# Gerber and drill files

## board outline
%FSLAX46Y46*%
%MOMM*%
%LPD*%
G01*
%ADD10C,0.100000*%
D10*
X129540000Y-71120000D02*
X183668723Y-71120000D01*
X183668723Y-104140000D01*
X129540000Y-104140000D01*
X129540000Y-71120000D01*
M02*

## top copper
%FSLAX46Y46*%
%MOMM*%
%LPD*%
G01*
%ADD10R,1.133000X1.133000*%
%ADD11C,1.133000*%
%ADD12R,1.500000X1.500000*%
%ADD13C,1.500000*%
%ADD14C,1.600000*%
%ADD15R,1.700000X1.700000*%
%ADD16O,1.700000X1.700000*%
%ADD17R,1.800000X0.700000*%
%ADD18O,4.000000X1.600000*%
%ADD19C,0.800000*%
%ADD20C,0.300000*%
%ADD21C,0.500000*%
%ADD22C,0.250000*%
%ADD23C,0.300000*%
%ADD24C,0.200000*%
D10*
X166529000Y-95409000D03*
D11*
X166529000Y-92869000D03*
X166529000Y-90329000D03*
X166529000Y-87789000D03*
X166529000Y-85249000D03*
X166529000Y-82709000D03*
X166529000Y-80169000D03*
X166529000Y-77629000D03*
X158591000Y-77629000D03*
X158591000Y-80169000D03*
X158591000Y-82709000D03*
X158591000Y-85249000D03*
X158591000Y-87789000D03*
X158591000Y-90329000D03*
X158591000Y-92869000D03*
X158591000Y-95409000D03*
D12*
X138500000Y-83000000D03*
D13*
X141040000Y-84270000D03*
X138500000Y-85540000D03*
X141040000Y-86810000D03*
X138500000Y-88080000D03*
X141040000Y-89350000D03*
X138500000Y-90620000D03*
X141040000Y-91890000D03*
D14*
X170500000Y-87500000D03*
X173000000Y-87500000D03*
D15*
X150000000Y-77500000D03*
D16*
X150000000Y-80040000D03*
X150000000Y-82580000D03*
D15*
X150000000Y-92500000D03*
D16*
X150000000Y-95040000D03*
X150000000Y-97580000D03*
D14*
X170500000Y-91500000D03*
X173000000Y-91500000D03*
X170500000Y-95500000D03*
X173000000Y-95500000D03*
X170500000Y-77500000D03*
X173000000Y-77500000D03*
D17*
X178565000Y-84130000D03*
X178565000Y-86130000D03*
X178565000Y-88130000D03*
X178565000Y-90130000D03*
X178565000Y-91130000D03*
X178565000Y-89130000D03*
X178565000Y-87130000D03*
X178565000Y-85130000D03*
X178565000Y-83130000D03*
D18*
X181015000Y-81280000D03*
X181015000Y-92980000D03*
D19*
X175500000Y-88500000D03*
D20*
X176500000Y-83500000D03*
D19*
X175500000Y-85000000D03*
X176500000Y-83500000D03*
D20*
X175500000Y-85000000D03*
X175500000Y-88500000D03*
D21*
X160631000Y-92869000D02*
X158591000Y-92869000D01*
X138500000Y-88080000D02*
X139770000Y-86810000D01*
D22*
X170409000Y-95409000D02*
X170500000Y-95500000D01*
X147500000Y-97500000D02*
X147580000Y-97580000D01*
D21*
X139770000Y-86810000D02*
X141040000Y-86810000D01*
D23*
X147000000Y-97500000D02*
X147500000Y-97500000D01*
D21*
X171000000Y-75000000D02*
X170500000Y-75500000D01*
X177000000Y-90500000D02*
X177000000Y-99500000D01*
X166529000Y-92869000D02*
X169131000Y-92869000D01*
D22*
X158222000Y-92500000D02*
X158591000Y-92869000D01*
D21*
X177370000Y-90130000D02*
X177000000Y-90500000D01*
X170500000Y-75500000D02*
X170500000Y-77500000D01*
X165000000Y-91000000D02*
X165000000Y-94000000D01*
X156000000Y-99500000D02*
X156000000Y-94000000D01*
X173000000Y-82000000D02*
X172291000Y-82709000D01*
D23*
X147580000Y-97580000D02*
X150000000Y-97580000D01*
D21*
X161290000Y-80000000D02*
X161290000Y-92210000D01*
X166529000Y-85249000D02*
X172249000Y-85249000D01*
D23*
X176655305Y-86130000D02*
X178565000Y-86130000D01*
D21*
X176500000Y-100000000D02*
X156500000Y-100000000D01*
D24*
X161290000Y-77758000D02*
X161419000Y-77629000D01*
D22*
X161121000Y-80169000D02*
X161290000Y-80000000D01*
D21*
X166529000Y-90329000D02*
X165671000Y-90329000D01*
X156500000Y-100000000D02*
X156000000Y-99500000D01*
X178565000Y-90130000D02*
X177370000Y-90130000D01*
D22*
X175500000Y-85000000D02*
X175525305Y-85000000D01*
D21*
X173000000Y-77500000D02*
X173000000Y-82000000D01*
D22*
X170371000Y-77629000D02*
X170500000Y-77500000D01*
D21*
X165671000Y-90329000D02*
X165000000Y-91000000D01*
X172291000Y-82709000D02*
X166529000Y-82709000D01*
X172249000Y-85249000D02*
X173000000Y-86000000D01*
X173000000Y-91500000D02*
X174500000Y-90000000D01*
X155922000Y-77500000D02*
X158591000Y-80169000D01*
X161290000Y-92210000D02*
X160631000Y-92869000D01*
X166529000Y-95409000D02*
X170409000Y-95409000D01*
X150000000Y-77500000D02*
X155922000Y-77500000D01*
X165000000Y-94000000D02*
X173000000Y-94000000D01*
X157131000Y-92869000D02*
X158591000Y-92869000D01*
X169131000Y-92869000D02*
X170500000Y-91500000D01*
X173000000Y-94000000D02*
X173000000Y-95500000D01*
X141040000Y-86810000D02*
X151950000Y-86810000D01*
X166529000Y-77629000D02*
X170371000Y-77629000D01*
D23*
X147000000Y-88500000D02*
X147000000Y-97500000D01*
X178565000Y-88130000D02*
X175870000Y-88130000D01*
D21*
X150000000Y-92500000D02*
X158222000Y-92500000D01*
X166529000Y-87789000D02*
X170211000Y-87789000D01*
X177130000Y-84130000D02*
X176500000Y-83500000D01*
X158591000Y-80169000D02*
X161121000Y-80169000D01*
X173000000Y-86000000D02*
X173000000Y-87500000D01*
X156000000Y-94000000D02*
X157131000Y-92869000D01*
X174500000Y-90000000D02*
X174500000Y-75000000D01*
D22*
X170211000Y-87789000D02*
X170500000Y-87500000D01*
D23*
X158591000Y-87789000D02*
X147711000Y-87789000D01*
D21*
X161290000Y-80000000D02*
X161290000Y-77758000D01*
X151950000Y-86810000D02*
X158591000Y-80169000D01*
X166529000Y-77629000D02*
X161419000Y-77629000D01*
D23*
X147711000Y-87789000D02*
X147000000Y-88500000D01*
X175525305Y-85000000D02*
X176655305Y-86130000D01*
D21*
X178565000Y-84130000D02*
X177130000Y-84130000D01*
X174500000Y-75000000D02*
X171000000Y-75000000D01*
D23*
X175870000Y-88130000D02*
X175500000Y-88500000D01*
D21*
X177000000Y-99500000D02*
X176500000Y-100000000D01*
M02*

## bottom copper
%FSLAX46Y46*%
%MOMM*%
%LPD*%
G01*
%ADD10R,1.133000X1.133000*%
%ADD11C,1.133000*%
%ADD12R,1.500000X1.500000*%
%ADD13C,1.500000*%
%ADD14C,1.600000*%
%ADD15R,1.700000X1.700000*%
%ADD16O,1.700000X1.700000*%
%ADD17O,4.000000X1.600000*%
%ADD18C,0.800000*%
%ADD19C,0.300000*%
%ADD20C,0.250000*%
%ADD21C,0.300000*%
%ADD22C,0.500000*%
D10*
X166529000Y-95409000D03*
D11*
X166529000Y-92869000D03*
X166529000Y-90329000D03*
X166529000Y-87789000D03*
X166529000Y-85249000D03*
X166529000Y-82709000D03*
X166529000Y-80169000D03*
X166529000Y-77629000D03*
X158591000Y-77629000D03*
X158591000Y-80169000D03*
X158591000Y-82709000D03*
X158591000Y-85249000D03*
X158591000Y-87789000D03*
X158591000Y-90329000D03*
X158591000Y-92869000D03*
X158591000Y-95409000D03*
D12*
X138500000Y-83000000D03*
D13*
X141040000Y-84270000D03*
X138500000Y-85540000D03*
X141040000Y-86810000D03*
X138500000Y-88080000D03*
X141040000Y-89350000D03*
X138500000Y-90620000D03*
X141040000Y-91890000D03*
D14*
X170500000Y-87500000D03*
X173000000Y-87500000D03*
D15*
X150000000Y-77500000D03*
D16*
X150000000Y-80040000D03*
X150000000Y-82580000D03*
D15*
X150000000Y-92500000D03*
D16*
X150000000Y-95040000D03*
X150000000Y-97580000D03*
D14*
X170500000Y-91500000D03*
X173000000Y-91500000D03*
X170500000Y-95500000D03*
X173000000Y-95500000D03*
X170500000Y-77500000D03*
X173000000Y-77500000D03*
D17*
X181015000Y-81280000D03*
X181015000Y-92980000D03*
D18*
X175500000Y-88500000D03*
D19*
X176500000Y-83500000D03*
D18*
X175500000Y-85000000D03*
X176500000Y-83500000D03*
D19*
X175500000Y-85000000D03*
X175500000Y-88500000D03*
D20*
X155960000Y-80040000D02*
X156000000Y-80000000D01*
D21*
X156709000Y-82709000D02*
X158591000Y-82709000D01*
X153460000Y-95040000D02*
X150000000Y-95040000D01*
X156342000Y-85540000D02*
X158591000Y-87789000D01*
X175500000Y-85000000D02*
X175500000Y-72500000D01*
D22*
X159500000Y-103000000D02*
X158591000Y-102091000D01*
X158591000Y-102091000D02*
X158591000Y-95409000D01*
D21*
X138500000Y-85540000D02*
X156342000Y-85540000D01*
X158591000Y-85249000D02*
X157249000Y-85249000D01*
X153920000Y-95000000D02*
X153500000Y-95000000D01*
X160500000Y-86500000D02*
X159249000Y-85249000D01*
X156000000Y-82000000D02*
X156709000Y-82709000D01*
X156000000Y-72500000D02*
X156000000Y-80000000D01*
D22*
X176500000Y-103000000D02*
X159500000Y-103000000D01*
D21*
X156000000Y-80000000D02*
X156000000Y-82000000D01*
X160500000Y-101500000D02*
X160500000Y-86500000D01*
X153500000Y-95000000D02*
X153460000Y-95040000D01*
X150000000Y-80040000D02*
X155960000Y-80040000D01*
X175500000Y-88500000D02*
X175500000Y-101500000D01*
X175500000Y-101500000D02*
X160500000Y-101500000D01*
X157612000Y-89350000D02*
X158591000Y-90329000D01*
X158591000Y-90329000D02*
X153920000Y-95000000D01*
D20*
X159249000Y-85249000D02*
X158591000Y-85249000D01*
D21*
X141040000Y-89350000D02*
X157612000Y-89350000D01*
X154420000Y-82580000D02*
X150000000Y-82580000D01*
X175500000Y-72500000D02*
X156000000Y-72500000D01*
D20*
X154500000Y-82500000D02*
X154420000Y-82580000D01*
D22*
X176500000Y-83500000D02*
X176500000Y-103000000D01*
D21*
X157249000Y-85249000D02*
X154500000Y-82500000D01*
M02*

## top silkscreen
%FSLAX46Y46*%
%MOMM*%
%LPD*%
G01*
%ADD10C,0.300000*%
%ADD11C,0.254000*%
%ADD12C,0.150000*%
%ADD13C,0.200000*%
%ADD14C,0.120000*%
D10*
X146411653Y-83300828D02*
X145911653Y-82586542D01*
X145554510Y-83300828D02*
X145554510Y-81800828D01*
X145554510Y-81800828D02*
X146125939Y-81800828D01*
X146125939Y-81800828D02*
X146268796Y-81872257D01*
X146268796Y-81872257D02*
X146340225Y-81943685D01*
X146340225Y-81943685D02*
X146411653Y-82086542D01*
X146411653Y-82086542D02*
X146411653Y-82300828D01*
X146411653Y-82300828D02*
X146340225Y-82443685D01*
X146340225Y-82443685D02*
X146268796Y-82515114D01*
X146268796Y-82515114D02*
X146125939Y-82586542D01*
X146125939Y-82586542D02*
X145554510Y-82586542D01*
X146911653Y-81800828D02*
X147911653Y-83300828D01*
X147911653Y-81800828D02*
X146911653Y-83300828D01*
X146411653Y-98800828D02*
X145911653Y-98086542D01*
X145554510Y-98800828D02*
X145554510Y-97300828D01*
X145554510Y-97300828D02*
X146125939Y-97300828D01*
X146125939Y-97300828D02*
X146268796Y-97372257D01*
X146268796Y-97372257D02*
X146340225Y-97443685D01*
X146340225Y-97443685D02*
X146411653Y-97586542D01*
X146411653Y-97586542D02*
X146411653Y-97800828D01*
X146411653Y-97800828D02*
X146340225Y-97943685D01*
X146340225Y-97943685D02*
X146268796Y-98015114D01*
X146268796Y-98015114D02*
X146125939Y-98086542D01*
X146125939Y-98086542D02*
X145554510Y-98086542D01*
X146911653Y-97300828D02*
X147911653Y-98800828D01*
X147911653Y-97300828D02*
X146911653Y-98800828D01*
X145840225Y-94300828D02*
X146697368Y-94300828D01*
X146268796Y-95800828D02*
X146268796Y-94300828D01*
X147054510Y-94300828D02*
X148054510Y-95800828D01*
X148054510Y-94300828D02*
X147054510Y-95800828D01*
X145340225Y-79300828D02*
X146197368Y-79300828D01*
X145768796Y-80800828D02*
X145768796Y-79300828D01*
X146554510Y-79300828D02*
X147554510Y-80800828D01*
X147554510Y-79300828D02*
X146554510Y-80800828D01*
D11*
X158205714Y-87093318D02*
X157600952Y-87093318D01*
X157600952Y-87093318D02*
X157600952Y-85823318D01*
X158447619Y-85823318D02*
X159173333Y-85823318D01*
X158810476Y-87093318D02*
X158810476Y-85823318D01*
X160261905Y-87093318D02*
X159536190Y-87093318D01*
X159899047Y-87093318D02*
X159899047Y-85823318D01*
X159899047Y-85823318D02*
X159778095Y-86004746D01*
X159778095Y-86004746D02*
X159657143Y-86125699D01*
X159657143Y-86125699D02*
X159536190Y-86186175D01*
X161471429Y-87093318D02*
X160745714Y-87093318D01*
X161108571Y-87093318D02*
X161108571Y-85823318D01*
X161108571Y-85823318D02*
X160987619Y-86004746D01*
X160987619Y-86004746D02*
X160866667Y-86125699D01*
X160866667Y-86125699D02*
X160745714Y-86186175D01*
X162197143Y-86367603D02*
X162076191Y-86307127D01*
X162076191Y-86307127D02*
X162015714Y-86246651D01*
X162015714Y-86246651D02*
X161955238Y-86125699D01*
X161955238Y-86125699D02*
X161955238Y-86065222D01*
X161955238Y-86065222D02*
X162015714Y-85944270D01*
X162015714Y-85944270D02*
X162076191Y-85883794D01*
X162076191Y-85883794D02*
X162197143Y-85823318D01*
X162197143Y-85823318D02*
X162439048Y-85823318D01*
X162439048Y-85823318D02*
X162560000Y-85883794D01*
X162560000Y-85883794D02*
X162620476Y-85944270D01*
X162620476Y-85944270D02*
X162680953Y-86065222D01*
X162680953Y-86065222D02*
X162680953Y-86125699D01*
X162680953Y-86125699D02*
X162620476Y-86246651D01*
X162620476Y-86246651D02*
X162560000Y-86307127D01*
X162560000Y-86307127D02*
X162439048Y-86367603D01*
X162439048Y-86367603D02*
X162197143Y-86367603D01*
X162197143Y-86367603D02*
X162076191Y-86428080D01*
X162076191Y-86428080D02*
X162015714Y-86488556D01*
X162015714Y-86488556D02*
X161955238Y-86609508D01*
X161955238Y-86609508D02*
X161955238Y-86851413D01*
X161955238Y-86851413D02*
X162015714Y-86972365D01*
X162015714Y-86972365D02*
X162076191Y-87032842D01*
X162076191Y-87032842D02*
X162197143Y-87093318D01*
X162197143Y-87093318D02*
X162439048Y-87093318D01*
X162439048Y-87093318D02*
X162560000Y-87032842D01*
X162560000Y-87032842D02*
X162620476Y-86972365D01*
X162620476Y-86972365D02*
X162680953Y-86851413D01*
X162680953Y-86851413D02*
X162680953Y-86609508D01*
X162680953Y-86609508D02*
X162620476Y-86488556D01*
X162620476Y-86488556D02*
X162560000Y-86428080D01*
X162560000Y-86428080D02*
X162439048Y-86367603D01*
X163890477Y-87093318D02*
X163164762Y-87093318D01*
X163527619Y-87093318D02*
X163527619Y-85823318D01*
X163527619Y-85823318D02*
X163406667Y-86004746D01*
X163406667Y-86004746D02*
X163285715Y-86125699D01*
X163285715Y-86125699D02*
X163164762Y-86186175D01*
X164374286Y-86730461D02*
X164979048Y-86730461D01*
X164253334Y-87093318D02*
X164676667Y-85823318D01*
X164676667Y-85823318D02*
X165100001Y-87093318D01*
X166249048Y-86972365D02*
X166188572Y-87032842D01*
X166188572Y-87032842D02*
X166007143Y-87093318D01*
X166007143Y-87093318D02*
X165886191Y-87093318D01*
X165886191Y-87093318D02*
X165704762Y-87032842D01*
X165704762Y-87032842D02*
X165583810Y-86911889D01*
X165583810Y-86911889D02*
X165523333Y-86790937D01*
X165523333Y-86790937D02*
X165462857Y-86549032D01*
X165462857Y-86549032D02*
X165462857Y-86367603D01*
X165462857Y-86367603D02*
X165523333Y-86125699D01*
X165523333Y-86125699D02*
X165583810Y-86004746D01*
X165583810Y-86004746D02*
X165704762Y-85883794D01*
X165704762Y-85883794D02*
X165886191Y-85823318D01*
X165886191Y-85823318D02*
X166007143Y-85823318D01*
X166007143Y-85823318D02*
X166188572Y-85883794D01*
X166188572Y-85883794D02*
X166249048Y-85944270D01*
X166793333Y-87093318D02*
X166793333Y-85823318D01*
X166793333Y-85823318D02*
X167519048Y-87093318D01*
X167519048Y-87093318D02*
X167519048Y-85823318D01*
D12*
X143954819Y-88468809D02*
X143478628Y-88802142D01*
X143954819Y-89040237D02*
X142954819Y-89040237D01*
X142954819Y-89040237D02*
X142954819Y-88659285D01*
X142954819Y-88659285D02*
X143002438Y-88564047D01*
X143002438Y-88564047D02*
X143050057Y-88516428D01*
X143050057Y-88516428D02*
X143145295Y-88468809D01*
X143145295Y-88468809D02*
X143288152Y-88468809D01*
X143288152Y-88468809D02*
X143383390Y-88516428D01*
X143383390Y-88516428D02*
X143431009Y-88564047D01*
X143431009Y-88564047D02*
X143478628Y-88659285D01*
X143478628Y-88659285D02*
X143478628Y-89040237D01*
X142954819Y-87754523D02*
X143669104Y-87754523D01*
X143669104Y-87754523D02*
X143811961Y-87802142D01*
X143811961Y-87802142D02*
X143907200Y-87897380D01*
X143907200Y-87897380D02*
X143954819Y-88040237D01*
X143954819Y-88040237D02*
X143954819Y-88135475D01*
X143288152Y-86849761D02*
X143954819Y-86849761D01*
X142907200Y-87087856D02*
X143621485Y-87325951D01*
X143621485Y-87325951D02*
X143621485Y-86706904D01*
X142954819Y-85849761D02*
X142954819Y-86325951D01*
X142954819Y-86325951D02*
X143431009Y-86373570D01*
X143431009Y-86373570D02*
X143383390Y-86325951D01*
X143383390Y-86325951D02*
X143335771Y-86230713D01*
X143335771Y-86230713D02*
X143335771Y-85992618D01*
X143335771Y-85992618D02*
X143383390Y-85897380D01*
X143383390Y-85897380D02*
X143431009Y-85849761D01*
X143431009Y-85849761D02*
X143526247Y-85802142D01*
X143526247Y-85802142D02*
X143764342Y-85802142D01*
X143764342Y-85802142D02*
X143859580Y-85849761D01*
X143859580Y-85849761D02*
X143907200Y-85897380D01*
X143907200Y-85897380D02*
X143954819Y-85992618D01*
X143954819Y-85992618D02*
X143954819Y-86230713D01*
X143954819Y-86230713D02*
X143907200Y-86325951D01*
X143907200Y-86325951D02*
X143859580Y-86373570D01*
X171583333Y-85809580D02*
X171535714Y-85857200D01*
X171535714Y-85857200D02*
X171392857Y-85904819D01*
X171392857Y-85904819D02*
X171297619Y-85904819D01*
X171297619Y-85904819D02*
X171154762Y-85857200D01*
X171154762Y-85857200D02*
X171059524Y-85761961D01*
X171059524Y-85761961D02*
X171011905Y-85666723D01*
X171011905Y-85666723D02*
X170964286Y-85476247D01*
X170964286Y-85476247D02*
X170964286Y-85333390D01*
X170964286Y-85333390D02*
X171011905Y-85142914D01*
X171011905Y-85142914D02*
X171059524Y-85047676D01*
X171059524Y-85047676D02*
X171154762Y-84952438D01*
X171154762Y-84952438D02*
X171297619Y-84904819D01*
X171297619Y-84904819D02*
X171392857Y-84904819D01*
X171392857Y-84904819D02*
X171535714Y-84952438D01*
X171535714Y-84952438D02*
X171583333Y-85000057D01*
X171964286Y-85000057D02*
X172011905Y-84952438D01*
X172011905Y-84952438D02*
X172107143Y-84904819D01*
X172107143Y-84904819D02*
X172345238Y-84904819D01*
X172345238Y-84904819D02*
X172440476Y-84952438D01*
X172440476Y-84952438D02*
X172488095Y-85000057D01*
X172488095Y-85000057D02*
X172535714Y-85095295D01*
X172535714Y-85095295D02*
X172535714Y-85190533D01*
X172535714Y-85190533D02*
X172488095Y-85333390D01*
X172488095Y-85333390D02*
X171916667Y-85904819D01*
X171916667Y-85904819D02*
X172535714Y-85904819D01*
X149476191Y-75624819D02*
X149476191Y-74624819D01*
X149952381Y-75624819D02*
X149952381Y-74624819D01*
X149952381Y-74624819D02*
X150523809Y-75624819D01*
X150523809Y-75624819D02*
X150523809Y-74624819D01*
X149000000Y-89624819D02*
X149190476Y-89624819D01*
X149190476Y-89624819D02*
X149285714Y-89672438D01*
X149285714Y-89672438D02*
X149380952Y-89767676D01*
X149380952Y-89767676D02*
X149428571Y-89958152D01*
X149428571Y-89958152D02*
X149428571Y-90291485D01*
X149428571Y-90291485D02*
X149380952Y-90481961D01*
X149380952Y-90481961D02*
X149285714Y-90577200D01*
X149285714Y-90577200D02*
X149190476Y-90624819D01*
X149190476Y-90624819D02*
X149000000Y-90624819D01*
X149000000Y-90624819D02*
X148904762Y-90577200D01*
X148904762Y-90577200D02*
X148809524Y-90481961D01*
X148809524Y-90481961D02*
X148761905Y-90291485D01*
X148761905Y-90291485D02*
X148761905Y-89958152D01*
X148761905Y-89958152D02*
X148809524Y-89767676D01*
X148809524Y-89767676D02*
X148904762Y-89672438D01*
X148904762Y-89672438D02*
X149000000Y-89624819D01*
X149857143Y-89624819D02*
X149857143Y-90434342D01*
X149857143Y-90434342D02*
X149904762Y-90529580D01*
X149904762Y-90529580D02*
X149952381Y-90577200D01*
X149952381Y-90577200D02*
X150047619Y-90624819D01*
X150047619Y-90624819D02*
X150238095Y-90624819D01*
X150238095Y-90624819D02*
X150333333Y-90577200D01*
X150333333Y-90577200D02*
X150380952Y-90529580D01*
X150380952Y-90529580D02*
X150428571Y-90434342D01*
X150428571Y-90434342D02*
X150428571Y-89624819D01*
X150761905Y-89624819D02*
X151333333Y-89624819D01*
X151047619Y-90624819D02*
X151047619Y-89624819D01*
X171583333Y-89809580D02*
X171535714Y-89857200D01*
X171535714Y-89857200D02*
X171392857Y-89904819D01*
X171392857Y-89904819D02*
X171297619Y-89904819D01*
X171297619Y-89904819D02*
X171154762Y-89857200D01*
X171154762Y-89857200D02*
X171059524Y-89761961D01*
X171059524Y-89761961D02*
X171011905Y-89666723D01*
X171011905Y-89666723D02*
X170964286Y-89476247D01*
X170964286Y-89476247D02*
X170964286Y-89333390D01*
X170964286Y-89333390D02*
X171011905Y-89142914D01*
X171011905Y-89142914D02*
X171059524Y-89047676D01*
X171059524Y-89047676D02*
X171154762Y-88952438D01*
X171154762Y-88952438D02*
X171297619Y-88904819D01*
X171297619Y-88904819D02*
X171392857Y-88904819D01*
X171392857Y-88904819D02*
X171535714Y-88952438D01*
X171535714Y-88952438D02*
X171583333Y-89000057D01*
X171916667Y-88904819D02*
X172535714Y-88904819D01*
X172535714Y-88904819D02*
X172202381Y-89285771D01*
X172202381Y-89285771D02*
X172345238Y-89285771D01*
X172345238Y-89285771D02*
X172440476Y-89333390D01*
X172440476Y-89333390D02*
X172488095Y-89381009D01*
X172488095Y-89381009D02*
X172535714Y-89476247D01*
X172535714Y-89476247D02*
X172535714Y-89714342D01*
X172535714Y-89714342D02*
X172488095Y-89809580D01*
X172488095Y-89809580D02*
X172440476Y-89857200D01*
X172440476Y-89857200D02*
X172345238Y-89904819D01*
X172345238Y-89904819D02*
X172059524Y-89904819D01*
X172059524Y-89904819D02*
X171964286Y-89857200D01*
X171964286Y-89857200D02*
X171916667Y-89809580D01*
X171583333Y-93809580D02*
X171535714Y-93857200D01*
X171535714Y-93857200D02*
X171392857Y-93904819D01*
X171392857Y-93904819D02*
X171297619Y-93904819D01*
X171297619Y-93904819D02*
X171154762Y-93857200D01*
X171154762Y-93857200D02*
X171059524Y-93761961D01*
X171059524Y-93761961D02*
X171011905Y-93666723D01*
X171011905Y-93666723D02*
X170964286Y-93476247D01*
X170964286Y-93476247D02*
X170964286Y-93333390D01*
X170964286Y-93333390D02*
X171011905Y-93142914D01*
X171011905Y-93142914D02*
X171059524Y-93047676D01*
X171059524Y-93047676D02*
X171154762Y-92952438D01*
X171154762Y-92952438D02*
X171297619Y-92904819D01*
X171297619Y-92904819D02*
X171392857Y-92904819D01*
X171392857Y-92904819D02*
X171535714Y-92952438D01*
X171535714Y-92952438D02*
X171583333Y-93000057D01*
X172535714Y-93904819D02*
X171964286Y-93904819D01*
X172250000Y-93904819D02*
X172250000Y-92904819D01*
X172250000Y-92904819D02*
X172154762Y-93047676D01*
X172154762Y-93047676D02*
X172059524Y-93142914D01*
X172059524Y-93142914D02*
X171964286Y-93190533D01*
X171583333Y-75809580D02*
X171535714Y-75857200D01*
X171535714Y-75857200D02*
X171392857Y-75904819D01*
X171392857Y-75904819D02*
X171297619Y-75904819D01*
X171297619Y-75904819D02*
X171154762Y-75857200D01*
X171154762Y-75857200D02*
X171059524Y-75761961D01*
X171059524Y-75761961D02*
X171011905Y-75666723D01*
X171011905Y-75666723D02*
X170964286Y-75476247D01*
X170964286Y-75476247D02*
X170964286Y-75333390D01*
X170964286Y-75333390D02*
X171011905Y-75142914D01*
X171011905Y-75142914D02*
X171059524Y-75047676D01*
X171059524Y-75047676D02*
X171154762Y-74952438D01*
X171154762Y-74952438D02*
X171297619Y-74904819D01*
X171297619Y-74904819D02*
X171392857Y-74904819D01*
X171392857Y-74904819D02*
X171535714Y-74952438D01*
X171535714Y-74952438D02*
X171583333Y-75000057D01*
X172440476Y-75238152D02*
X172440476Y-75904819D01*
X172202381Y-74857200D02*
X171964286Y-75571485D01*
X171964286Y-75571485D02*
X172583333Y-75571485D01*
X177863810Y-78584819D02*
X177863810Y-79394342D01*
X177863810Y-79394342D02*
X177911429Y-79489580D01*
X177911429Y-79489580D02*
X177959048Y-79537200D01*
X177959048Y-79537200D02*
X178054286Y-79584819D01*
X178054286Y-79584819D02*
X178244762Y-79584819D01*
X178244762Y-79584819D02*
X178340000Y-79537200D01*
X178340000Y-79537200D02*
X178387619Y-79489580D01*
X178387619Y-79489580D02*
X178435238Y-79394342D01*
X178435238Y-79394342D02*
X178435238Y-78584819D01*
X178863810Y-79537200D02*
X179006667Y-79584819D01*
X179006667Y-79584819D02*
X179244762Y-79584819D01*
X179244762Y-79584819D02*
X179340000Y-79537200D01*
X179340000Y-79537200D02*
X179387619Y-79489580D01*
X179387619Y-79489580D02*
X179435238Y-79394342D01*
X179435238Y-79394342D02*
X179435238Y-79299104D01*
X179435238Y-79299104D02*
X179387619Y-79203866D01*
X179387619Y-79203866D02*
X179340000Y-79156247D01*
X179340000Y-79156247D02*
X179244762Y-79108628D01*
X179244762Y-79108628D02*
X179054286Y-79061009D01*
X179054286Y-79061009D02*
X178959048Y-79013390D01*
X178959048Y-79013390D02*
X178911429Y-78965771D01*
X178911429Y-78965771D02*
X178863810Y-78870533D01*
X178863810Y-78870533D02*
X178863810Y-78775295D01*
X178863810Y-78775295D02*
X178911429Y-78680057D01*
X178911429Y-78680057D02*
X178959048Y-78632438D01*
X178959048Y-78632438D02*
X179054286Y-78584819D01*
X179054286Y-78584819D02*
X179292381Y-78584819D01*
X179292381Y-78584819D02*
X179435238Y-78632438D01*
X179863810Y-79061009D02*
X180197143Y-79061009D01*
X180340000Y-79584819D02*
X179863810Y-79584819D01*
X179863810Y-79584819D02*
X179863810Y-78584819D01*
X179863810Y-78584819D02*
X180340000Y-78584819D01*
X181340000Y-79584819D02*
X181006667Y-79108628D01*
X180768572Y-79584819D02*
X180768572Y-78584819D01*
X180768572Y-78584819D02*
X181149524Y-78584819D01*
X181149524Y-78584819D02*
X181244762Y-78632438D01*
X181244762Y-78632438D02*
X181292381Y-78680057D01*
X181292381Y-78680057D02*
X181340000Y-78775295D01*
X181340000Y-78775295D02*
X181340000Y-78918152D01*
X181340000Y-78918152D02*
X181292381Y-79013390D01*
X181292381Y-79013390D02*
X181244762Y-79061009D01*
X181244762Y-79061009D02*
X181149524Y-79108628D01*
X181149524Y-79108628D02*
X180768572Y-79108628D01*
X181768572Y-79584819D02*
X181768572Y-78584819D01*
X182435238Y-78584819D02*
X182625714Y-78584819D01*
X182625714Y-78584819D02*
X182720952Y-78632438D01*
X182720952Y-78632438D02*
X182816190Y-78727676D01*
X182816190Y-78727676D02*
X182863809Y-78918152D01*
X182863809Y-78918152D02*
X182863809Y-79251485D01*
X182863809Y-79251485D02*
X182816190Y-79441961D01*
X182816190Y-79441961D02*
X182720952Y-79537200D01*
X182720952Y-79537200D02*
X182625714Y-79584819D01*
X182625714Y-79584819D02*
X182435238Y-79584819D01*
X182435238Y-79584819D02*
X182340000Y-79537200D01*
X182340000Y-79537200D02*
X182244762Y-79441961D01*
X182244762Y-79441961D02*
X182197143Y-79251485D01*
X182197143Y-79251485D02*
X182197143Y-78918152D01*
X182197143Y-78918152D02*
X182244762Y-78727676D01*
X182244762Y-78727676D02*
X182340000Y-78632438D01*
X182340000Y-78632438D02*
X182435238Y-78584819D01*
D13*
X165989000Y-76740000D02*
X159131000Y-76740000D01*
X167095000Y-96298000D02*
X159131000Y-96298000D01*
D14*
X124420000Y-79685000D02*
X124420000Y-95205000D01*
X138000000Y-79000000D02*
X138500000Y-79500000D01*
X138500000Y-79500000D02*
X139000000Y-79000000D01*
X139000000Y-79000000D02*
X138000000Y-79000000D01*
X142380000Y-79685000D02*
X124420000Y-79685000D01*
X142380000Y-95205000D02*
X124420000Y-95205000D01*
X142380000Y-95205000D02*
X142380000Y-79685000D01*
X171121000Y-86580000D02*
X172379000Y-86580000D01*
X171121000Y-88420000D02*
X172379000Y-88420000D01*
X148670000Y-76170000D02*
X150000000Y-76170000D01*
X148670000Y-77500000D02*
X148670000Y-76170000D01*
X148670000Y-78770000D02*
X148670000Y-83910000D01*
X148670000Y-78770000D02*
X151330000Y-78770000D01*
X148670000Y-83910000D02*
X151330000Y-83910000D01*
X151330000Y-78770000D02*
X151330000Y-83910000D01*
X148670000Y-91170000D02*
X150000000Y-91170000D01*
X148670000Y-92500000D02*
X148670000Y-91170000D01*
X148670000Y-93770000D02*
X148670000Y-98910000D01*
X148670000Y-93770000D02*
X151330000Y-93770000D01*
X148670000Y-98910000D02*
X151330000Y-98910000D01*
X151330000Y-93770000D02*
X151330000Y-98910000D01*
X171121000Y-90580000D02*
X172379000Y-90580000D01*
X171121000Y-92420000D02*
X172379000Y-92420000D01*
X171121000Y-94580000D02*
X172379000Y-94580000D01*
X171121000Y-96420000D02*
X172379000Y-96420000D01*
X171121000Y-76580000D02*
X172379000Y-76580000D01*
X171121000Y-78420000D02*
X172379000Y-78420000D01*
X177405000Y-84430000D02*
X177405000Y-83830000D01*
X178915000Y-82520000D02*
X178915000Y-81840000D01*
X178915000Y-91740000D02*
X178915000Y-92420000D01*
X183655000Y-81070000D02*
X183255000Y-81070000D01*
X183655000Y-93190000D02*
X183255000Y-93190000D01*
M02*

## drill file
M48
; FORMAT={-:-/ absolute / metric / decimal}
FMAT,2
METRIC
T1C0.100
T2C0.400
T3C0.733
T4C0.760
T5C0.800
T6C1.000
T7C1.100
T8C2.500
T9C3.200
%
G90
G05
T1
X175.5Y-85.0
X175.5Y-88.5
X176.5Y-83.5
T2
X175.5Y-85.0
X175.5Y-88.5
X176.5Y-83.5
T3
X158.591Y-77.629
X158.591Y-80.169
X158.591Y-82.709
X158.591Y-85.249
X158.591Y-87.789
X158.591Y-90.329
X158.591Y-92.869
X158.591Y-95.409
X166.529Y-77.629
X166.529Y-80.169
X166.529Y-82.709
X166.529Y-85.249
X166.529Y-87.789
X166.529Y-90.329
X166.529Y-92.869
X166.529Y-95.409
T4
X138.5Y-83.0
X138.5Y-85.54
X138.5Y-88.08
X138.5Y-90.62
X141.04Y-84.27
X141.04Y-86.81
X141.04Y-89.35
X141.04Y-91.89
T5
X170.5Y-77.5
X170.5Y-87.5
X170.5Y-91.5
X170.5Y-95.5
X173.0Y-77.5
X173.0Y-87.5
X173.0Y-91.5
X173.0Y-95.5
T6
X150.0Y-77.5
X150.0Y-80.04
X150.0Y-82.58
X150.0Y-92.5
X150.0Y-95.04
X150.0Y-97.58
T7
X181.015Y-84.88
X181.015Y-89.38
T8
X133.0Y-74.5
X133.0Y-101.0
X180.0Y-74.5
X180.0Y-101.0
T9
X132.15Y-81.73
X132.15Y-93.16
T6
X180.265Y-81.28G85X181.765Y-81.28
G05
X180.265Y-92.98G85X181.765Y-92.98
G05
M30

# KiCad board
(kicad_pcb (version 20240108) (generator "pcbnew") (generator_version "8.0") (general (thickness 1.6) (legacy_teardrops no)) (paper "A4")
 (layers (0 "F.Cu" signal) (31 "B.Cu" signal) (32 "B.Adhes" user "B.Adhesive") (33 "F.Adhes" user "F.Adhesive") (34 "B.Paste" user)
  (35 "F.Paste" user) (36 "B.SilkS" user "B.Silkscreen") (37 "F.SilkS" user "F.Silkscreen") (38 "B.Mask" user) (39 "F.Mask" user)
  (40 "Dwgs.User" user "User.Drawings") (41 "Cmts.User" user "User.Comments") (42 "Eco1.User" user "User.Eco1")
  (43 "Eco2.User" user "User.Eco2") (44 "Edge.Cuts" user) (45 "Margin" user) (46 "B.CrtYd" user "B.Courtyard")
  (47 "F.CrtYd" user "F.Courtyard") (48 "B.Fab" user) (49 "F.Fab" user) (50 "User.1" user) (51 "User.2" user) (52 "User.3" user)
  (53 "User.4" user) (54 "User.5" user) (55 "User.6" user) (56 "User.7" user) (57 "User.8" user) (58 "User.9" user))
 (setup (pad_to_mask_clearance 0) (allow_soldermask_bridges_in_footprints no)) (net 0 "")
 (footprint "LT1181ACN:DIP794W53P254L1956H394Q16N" (layer "F.Cu") (at 162.56 86.519 180)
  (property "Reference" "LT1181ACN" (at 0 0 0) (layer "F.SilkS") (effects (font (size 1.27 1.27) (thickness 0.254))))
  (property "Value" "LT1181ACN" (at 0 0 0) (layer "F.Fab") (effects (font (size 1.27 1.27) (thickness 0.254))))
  (fp_line (start -3.429 9.779) (end 3.429 9.779) (stroke (width 0.2) (type solid)) (layer "F.SilkS"))
  (fp_line (start -4.535 -9.779) (end 3.429 -9.779) (stroke (width 0.2) (type solid)) (layer "F.SilkS"))
  (pad "1" thru_hole rect (at -3.969 -8.89 180) (size 1.133 1.133) (drill 0.733) (layers "*.Cu" "*.Mask") (remove_unused_layers no))
  (pad "2" thru_hole circle (at -3.969 -6.35 180) (size 1.133 1.133) (drill 0.733) (layers "*.Cu" "*.Mask") (remove_unused_layers no))
  (pad "3" thru_hole circle (at -3.969 -3.81 180) (size 1.133 1.133) (drill 0.733) (layers "*.Cu" "*.Mask") (remove_unused_layers no))
  (pad "4" thru_hole circle (at -3.969 -1.27 180) (size 1.133 1.133) (drill 0.733) (layers "*.Cu" "*.Mask") (remove_unused_layers no))
  (pad "5" thru_hole circle (at -3.969 1.27 180) (size 1.133 1.133) (drill 0.733) (layers "*.Cu" "*.Mask") (remove_unused_layers no))
  (pad "6" thru_hole circle (at -3.969 3.81 180) (size 1.133 1.133) (drill 0.733) (layers "*.Cu" "*.Mask") (remove_unused_layers no))
  (pad "7" thru_hole circle (at -3.969 6.35 180) (size 1.133 1.133) (drill 0.733) (layers "*.Cu" "*.Mask") (remove_unused_layers no))
  (pad "8" thru_hole circle (at -3.969 8.89 180) (size 1.133 1.133) (drill 0.733) (layers "*.Cu" "*.Mask") (remove_unused_layers no))
  (pad "9" thru_hole circle (at 3.969 8.89 180) (size 1.133 1.133) (drill 0.733) (layers "*.Cu" "*.Mask") (remove_unused_layers no))
  (pad "10" thru_hole circle (at 3.969 6.35 180) (size 1.133 1.133) (drill 0.733) (layers "*.Cu" "*.Mask") (remove_unused_layers no))
  (pad "11" thru_hole circle (at 3.969 3.81 180) (size 1.133 1.133) (drill 0.733) (layers "*.Cu" "*.Mask") (remove_unused_layers no))
  (pad "12" thru_hole circle (at 3.969 1.27 180) (size 1.133 1.133) (drill 0.733) (layers "*.Cu" "*.Mask") (remove_unused_layers no))
  (pad "13" thru_hole circle (at 3.969 -1.27 180) (size 1.133 1.133) (drill 0.733) (layers "*.Cu" "*.Mask") (remove_unused_layers no))
  (pad "14" thru_hole circle (at 3.969 -3.81 180) (size 1.133 1.133) (drill 0.733) (layers "*.Cu" "*.Mask") (remove_unused_layers no))
  (pad "15" thru_hole circle (at 3.969 -6.35 180) (size 1.133 1.133) (drill 0.733) (layers "*.Cu" "*.Mask") (remove_unused_layers no))
  (pad "16" thru_hole circle (at 3.969 -8.89 180) (size 1.133 1.133) (drill 0.733) (layers "*.Cu" "*.Mask") (remove_unused_layers no)))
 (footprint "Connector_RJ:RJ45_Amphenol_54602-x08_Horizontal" (layer "F.Cu") (at 138.5 83 -90)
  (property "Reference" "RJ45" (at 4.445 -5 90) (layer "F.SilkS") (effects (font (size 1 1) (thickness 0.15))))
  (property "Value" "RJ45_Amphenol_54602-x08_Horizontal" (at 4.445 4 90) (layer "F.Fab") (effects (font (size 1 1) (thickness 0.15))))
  (fp_line (start -3.315 14.08) (end 12.205 14.08) (stroke (width 0.12) (type solid)) (layer "F.SilkS"))
  (fp_line (start -4 0.5) (end -3.5 0) (stroke (width 0.12) (type solid)) (layer "F.SilkS"))
  (fp_line (start -3.5 0) (end -4 -0.5) (stroke (width 0.12) (type solid)) (layer "F.SilkS"))
  (fp_line (start -4 -0.5) (end -4 0.5) (stroke (width 0.12) (type solid)) (layer "F.SilkS"))
  (fp_line (start -3.315 -3.88) (end -3.315 14.08) (stroke (width 0.12) (type solid)) (layer "F.SilkS"))
  (fp_line (start 12.205 -3.88) (end 12.205 14.08) (stroke (width 0.12) (type solid)) (layer "F.SilkS"))
  (fp_line (start 12.205 -3.88) (end -3.315 -3.88) (stroke (width 0.12) (type solid)) (layer "F.SilkS"))
  (pad "" np_thru_hole circle (at -1.27 6.35 270) (size 3.2 3.2) (drill 3.2) (layers "*.Cu" "*.Mask"))
  (pad "" np_thru_hole circle (at 10.16 6.35 270) (size 3.2 3.2) (drill 3.2) (layers "*.Cu" "*.Mask"))
  (pad "1" thru_hole rect (at 0 0 270) (size 1.5 1.5) (drill 0.76) (layers "*.Cu" "*.Mask") (remove_unused_layers no))
  (pad "2" thru_hole circle (at 1.27 -2.54 270) (size 1.5 1.5) (drill 0.76) (layers "*.Cu" "*.Mask") (remove_unused_layers no))
  (pad "3" thru_hole circle (at 2.54 0 270) (size 1.5 1.5) (drill 0.76) (layers "*.Cu" "*.Mask") (remove_unused_layers no))
  (pad "4" thru_hole circle (at 3.81 -2.54 270) (size 1.5 1.5) (drill 0.76) (layers "*.Cu" "*.Mask") (remove_unused_layers no))
  (pad "5" thru_hole circle (at 5.08 0 270) (size 1.5 1.5) (drill 0.76) (layers "*.Cu" "*.Mask") (remove_unused_layers no))
  (pad "6" thru_hole circle (at 6.35 -2.54 270) (size 1.5 1.5) (drill 0.76) (layers "*.Cu" "*.Mask") (remove_unused_layers no))
  (pad "7" thru_hole circle (at 7.62 0 270) (size 1.5 1.5) (drill 0.76) (layers "*.Cu" "*.Mask") (remove_unused_layers no))
  (pad "8" thru_hole circle (at 8.89 -2.54 270) (size 1.5 1.5) (drill 0.76) (layers "*.Cu" "*.Mask") (remove_unused_layers no)))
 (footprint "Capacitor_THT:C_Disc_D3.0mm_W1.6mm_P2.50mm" (layer "F.Cu") (at 170.5 87.5)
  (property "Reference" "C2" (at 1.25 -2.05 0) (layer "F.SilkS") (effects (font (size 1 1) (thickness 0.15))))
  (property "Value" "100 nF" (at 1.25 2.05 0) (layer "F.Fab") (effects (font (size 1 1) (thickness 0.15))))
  (fp_line (start 0.621 -0.92) (end 1.879 -0.92) (stroke (width 0.12) (type solid)) (layer "F.SilkS"))
  (fp_line (start 0.621 0.92) (end 1.879 0.92) (stroke (width 0.12) (type solid)) (layer "F.SilkS"))
  (pad "1" thru_hole circle (at 0 0) (size 1.6 1.6) (drill 0.8) (layers "*.Cu" "*.Mask") (remove_unused_layers no))
  (pad "2" thru_hole circle (at 2.5 0) (size 1.6 1.6) (drill 0.8) (layers "*.Cu" "*.Mask") (remove_unused_layers no)))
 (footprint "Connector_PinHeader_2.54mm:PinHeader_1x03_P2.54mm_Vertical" (layer "F.Cu") (at 150 77.5)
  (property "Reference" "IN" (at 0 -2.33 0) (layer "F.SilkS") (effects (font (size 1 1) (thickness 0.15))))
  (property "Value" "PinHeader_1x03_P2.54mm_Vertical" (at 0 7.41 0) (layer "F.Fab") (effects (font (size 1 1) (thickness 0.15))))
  (fp_line (start -1.33 -1.33) (end 0 -1.33) (stroke (width 0.12) (type solid)) (layer "F.SilkS"))
  (fp_line (start -1.33 0) (end -1.33 -1.33) (stroke (width 0.12) (type solid)) (layer "F.SilkS"))
  (fp_line (start -1.33 1.27) (end -1.33 6.41) (stroke (width 0.12) (type solid)) (layer "F.SilkS"))
  (fp_line (start -1.33 1.27) (end 1.33 1.27) (stroke (width 0.12) (type solid)) (layer "F.SilkS"))
  (fp_line (start -1.33 6.41) (end 1.33 6.41) (stroke (width 0.12) (type solid)) (layer "F.SilkS"))
  (fp_line (start 1.33 1.27) (end 1.33 6.41) (stroke (width 0.12) (type solid)) (layer "F.SilkS"))
  (pad "1" thru_hole rect (at 0 0) (size 1.7 1.7) (drill 1) (layers "*.Cu" "*.Mask") (remove_unused_layers no))
  (pad "2" thru_hole oval (at 0 2.54) (size 1.7 1.7) (drill 1) (layers "*.Cu" "*.Mask") (remove_unused_layers no))
  (pad "3" thru_hole oval (at 0 5.08) (size 1.7 1.7) (drill 1) (layers "*.Cu" "*.Mask") (remove_unused_layers no)))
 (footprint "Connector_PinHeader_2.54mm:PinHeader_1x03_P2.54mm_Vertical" (layer "F.Cu") (at 150 92.5)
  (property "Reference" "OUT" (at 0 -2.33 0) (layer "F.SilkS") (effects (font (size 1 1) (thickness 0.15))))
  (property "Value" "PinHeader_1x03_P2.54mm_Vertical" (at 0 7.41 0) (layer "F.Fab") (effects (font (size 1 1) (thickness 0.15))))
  (fp_line (start -1.33 -1.33) (end 0 -1.33) (stroke (width 0.12) (type solid)) (layer "F.SilkS"))
  (fp_line (start -1.33 0) (end -1.33 -1.33) (stroke (width 0.12) (type solid)) (layer "F.SilkS"))
  (fp_line (start -1.33 1.27) (end -1.33 6.41) (stroke (width 0.12) (type solid)) (layer "F.SilkS"))
  (fp_line (start -1.33 1.27) (end 1.33 1.27) (stroke (width 0.12) (type solid)) (layer "F.SilkS"))
  (fp_line (start -1.33 6.41) (end 1.33 6.41) (stroke (width 0.12) (type solid)) (layer "F.SilkS"))
  (fp_line (start 1.33 1.27) (end 1.33 6.41) (stroke (width 0.12) (type solid)) (layer "F.SilkS"))
  (pad "1" thru_hole rect (at 0 0) (size 1.7 1.7) (drill 1) (layers "*.Cu" "*.Mask") (remove_unused_layers no))
  (pad "2" thru_hole oval (at 0 2.54) (size 1.7 1.7) (drill 1) (layers "*.Cu" "*.Mask") (remove_unused_layers no))
  (pad "3" thru_hole oval (at 0 5.08) (size 1.7 1.7) (drill 1) (layers "*.Cu" "*.Mask") (remove_unused_layers no)))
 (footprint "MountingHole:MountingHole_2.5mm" (layer "F.Cu") (at 180 74.5)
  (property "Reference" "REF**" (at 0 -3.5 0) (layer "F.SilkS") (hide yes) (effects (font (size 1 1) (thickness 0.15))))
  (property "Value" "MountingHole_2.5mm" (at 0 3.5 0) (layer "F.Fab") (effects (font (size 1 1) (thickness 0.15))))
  (pad "" np_thru_hole circle (at 0 0) (size 2.5 2.5) (drill 2.5) (layers "*.Cu" "*.Mask")))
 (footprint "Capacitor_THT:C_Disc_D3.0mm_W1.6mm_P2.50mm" (layer "F.Cu") (at 170.5 91.5)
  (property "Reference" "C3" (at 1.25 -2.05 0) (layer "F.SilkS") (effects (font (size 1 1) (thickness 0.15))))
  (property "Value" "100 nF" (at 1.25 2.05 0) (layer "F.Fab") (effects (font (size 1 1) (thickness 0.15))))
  (fp_line (start 0.621 -0.92) (end 1.879 -0.92) (stroke (width 0.12) (type solid)) (layer "F.SilkS"))
  (fp_line (start 0.621 0.92) (end 1.879 0.92) (stroke (width 0.12) (type solid)) (layer "F.SilkS"))
  (pad "1" thru_hole circle (at 0 0) (size 1.6 1.6) (drill 0.8) (layers "*.Cu" "*.Mask") (remove_unused_layers no))
  (pad "2" thru_hole circle (at 2.5 0) (size 1.6 1.6) (drill 0.8) (layers "*.Cu" "*.Mask") (remove_unused_layers no)))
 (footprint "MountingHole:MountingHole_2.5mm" (layer "F.Cu") (at 133 101)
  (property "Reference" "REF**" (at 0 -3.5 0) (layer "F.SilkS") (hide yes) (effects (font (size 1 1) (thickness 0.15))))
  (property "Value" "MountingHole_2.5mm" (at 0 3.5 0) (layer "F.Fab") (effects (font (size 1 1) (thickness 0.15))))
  (pad "" np_thru_hole circle (at 0 0) (size 2.5 2.5) (drill 2.5) (layers "*.Cu" "*.Mask")))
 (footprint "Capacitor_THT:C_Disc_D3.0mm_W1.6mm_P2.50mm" (layer "F.Cu") (at 170.5 95.5)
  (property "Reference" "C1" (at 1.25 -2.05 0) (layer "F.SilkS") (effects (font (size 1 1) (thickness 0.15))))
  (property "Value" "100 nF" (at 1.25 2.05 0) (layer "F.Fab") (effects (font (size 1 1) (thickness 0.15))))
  (fp_line (start 0.621 -0.92) (end 1.879 -0.92) (stroke (width 0.12) (type solid)) (layer "F.SilkS"))
  (fp_line (start 0.621 0.92) (end 1.879 0.92) (stroke (width 0.12) (type solid)) (layer "F.SilkS"))
  (pad "1" thru_hole circle (at 0 0) (size 1.6 1.6) (drill 0.8) (layers "*.Cu" "*.Mask") (remove_unused_layers no))
  (pad "2" thru_hole circle (at 2.5 0) (size 1.6 1.6) (drill 0.8) (layers "*.Cu" "*.Mask") (remove_unused_layers no)))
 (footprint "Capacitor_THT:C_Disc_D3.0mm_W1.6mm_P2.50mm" (layer "F.Cu") (at 170.5 77.5)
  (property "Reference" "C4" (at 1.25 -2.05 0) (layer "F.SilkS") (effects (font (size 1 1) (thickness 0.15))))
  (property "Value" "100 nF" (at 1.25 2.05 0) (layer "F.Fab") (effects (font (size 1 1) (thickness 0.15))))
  (fp_line (start 0.621 -0.92) (end 1.879 -0.92) (stroke (width 0.12) (type solid)) (layer "F.SilkS"))
  (fp_line (start 0.621 0.92) (end 1.879 0.92) (stroke (width 0.12) (type solid)) (layer "F.SilkS"))
  (pad "1" thru_hole circle (at 0 0) (size 1.6 1.6) (drill 0.8) (layers "*.Cu" "*.Mask") (remove_unused_layers no))
  (pad "2" thru_hole circle (at 2.5 0) (size 1.6 1.6) (drill 0.8) (layers "*.Cu" "*.Mask") (remove_unused_layers no)))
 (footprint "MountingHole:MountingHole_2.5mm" (layer "F.Cu") (at 133 74.5)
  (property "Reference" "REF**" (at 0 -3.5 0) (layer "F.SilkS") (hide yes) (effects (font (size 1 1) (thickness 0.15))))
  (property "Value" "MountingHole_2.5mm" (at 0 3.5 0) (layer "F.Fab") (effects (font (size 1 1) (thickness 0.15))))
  (pad "" np_thru_hole circle (at 0 0) (size 2.5 2.5) (drill 2.5) (layers "*.Cu" "*.Mask")))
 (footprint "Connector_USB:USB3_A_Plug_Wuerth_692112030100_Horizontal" (layer "F.Cu") (at 180.34 87.13)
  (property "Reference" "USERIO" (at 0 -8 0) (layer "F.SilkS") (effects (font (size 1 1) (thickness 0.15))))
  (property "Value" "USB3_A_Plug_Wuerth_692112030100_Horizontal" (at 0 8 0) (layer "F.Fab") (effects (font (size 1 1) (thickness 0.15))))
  (fp_line (start -2.935 -2.7) (end -2.935 -3.3) (stroke (width 0.12) (type solid)) (layer "F.SilkS"))
  (fp_line (start -1.425 -4.61) (end -1.425 -5.29) (stroke (width 0.12) (type solid)) (layer "F.SilkS"))
  (fp_line (start -1.425 4.61) (end -1.425 5.29) (stroke (width 0.12) (type solid)) (layer "F.SilkS"))
  (fp_line (start 3.315 -6.06) (end 2.915 -6.06) (stroke (width 0.12) (type solid)) (layer "F.SilkS"))
  (fp_line (start 3.315 6.06) (end 2.915 6.06) (stroke (width 0.12) (type solid)) (layer "F.SilkS"))
  (pad "" np_thru_hole circle (at 0.675 -2.25 90) (size 1.1 1.1) (drill 1.1) (layers "*.Cu" "*.Mask"))
  (pad "" np_thru_hole circle (at 0.675 2.25 90) (size 1.1 1.1) (drill 1.1) (layers "*.Cu" "*.Mask"))
  (pad "1" smd rect (at -1.775 -3 90) (size 0.7 1.8) (layers "F.Cu" "F.Paste" "F.Mask"))
  (pad "2" smd rect (at -1.775 -1 90) (size 0.7 1.8) (layers "F.Cu" "F.Paste" "F.Mask"))
  (pad "3" smd rect (at -1.775 1 90) (size 0.7 1.8) (layers "F.Cu" "F.Paste" "F.Mask"))
  (pad "4" smd rect (at -1.775 3 90) (size 0.7 1.8) (layers "F.Cu" "F.Paste" "F.Mask"))
  (pad "5" smd rect (at -1.775 4 90) (size 0.7 1.8) (layers "F.Cu" "F.Paste" "F.Mask"))
  (pad "6" smd rect (at -1.775 2 90) (size 0.7 1.8) (layers "F.Cu" "F.Paste" "F.Mask"))
  (pad "7" smd rect (at -1.775 0 90) (size 0.7 1.8) (layers "F.Cu" "F.Paste" "F.Mask"))
  (pad "8" smd rect (at -1.775 -2 90) (size 0.7 1.8) (layers "F.Cu" "F.Paste" "F.Mask"))
  (pad "9" smd rect (at -1.775 -4) (size 1.8 0.7) (layers "F.Cu" "F.Paste" "F.Mask"))
  (pad "10" thru_hole oval (at 0.675 -5.85 90) (size 1.6 4) (drill oval 1 2.5) (layers "*.Cu" "*.Mask") (remove_unused_layers no))
  (pad "10" thru_hole oval (at 0.675 5.85 90) (size 1.6 4) (drill oval 1 2.5) (layers "*.Cu" "*.Mask") (remove_unused_layers no)))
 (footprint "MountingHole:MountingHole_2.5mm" (layer "F.Cu") (at 180 101)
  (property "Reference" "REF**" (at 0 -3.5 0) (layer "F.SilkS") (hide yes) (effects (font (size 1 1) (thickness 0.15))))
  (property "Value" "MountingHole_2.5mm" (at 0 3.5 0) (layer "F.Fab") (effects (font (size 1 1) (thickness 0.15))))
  (pad "" np_thru_hole circle (at 0 0) (size 2.5 2.5) (drill 2.5) (layers "*.Cu" "*.Mask")))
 (gr_rect (start 129.54 71.12) (end 183.668723 104.14) (stroke (width 0.1) (type solid)) (fill none) (layer "Edge.Cuts"))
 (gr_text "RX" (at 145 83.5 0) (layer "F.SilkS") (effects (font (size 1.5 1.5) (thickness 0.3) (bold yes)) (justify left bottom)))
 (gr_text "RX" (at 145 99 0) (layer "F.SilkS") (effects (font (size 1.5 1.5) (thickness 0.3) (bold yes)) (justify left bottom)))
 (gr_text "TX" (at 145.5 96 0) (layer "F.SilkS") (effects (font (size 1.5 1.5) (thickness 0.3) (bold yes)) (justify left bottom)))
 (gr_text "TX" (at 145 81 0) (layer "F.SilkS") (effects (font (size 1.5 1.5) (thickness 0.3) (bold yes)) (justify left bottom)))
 (segment (start 160.631 92.869) (end 158.591 92.869) (width 0.5) (layer "F.Cu") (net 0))
 (segment (start 138.5 88.08) (end 139.77 86.81) (width 0.5) (layer "F.Cu") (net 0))
 (segment (start 170.409 95.409) (end 170.5 95.5) (width 0.25) (layer "F.Cu") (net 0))
 (segment (start 147.5 97.5) (end 147.58 97.58) (width 0.25) (layer "F.Cu") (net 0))
 (segment (start 139.77 86.81) (end 141.04 86.81) (width 0.5) (layer "F.Cu") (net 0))
 (segment (start 147 97.5) (end 147.5 97.5) (width 0.3) (layer "F.Cu") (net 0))
 (segment (start 171 75) (end 170.5 75.5) (width 0.5) (layer "F.Cu") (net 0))
 (segment (start 177 90.5) (end 177 99.5) (width 0.5) (layer "F.Cu") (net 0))
 (segment (start 166.529 92.869) (end 169.131 92.869) (width 0.5) (layer "F.Cu") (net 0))
 (segment (start 158.222 92.5) (end 158.591 92.869) (width 0.25) (layer "F.Cu") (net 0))
 (segment (start 177.37 90.13) (end 177 90.5) (width 0.5) (layer "F.Cu") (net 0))
 (segment (start 170.5 75.5) (end 170.5 77.5) (width 0.5) (layer "F.Cu") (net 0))
 (segment (start 165 91) (end 165 94) (width 0.5) (layer "F.Cu") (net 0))
 (segment (start 156 99.5) (end 156 94) (width 0.5) (layer "F.Cu") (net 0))
 (segment (start 173 82) (end 172.291 82.709) (width 0.5) (layer "F.Cu") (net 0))
 (segment (start 147.58 97.58) (end 150 97.58) (width 0.3) (layer "F.Cu") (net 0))
 (segment (start 161.29 80) (end 161.29 92.21) (width 0.5) (layer "F.Cu") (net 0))
 (segment (start 166.529 85.249) (end 172.249 85.249) (width 0.5) (layer "F.Cu") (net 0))
 (segment (start 176.655305 86.13) (end 178.565 86.13) (width 0.3) (layer "F.Cu") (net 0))
 (segment (start 176.5 100) (end 156.5 100) (width 0.5) (layer "F.Cu") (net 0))
 (segment (start 161.29 77.758) (end 161.419 77.629) (width 0.2) (layer "F.Cu") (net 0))
 (segment (start 161.121 80.169) (end 161.29 80) (width 0.25) (layer "F.Cu") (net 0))
 (segment (start 166.529 90.329) (end 165.671 90.329) (width 0.5) (layer "F.Cu") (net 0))
 (segment (start 156.5 100) (end 156 99.5) (width 0.5) (layer "F.Cu") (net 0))
 (segment (start 178.565 90.13) (end 177.37 90.13) (width 0.5) (layer "F.Cu") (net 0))
 (segment (start 175.5 85) (end 175.525305 85) (width 0.25) (layer "F.Cu") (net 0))
 (segment (start 173 77.5) (end 173 82) (width 0.5) (layer "F.Cu") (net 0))
 (segment (start 170.371 77.629) (end 170.5 77.5) (width 0.25) (layer "F.Cu") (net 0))
 (segment (start 165.671 90.329) (end 165 91) (width 0.5) (layer "F.Cu") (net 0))
 (segment (start 172.291 82.709) (end 166.529 82.709) (width 0.5) (layer "F.Cu") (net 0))
 (segment (start 172.249 85.249) (end 173 86) (width 0.5) (layer "F.Cu") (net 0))
 (segment (start 173 91.5) (end 174.5 90) (width 0.5) (layer "F.Cu") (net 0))
 (segment (start 155.922 77.5) (end 158.591 80.169) (width 0.5) (layer "F.Cu") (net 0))
 (segment (start 161.29 92.21) (end 160.631 92.869) (width 0.5) (layer "F.Cu") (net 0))
 (segment (start 166.529 95.409) (end 170.409 95.409) (width 0.5) (layer "F.Cu") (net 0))
 (segment (start 150 77.5) (end 155.922 77.5) (width 0.5) (layer "F.Cu") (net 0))
 (segment (start 165 94) (end 173 94) (width 0.5) (layer "F.Cu") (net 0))
 (segment (start 157.131 92.869) (end 158.591 92.869) (width 0.5) (layer "F.Cu") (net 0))
 (segment (start 169.131 92.869) (end 170.5 91.5) (width 0.5) (layer "F.Cu") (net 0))
 (segment (start 173 94) (end 173 95.5) (width 0.5) (layer "F.Cu") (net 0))
 (segment (start 141.04 86.81) (end 151.95 86.81) (width 0.5) (layer "F.Cu") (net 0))
 (segment (start 166.529 77.629) (end 170.371 77.629) (width 0.5) (layer "F.Cu") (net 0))
 (segment (start 147 88.5) (end 147 97.5) (width 0.3) (layer "F.Cu") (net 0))
 (segment (start 178.565 88.13) (end 175.87 88.13) (width 0.3) (layer "F.Cu") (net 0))
 (segment (start 150 92.5) (end 158.222 92.5) (width 0.5) (layer "F.Cu") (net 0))
 (segment (start 166.529 87.789) (end 170.211 87.789) (width 0.5) (layer "F.Cu") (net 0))
 (segment (start 177.13 84.13) (end 176.5 83.5) (width 0.5) (layer "F.Cu") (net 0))
 (segment (start 158.591 80.169) (end 161.121 80.169) (width 0.5) (layer "F.Cu") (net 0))
 (segment (start 173 86) (end 173 87.5) (width 0.5) (layer "F.Cu") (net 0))
 (segment (start 156 94) (end 157.131 92.869) (width 0.5) (layer "F.Cu") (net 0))
 (segment (start 174.5 90) (end 174.5 75) (width 0.5) (layer "F.Cu") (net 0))
 (segment (start 170.211 87.789) (end 170.5 87.5) (width 0.25) (layer "F.Cu") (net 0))
 (segment (start 158.591 87.789) (end 147.711 87.789) (width 0.3) (layer "F.Cu") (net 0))
 (segment (start 161.29 80) (end 161.29 77.758) (width 0.5) (layer "F.Cu") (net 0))
 (segment (start 151.95 86.81) (end 158.591 80.169) (width 0.5) (layer "F.Cu") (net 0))
 (segment (start 166.529 77.629) (end 161.419 77.629) (width 0.5) (layer "F.Cu") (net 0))
 (segment (start 147.711 87.789) (end 147 88.5) (width 0.3) (layer "F.Cu") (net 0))
 (segment (start 175.525305 85) (end 176.655305 86.13) (width 0.3) (layer "F.Cu") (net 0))
 (segment (start 178.565 84.13) (end 177.13 84.13) (width 0.5) (layer "F.Cu") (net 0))
 (segment (start 174.5 75) (end 171 75) (width 0.5) (layer "F.Cu") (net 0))
 (segment (start 175.87 88.13) (end 175.5 88.5) (width 0.3) (layer "F.Cu") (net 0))
 (segment (start 177 99.5) (end 176.5 100) (width 0.5) (layer "F.Cu") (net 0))
 (via (at 175.5 88.5) (size 0.8) (drill 0.4) (layers "F.Cu" "B.Cu") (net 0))
 (via micro (at 176.5 83.5) (size 0.3) (drill 0.1) (layers "F.Cu" "B.Cu") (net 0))
 (via (at 175.5 85) (size 0.8) (drill 0.4) (layers "F.Cu" "B.Cu") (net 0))
 (via (at 176.5 83.5) (size 0.8) (drill 0.4) (layers "F.Cu" "B.Cu") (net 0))
 (via micro (at 175.5 85) (size 0.3) (drill 0.1) (layers "F.Cu" "B.Cu") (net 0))
 (via micro (at 175.5 88.5) (size 0.3) (drill 0.1) (layers "F.Cu" "B.Cu") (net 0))
 (segment (start 155.96 80.04) (end 156 80) (width 0.25) (layer "B.Cu") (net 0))
 (segment (start 156.709 82.709) (end 158.591 82.709) (width 0.3) (layer "B.Cu") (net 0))
 (segment (start 153.46 95.04) (end 150 95.04) (width 0.3) (layer "B.Cu") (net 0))
 (segment (start 156.342 85.54) (end 158.591 87.789) (width 0.3) (layer "B.Cu") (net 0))
 (segment (start 175.5 85) (end 175.5 72.5) (width 0.3) (layer "B.Cu") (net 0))
 (segment (start 159.5 103) (end 158.591 102.091) (width 0.5) (layer "B.Cu") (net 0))
 (segment (start 158.591 102.091) (end 158.591 95.409) (width 0.5) (layer "B.Cu") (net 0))
 (segment (start 138.5 85.54) (end 156.342 85.54) (width 0.3) (layer "B.Cu") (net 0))
 (segment (start 158.591 85.249) (end 157.249 85.249) (width 0.3) (layer "B.Cu") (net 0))
 (segment (start 153.92 95) (end 153.5 95) (width 0.3) (layer "B.Cu") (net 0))
 (segment (start 160.5 86.5) (end 159.249 85.249) (width 0.3) (layer "B.Cu") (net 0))
 (segment (start 156 82) (end 156.709 82.709) (width 0.3) (layer "B.Cu") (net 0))
 (segment (start 156 72.5) (end 156 80) (width 0.3) (layer "B.Cu") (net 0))
 (segment (start 176.5 103) (end 159.5 103) (width 0.5) (layer "B.Cu") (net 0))
 (segment (start 156 80) (end 156 82) (width 0.3) (layer "B.Cu") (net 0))
 (segment (start 160.5 101.5) (end 160.5 86.5) (width 0.3) (layer "B.Cu") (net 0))
 (segment (start 153.5 95) (end 153.46 95.04) (width 0.3) (layer "B.Cu") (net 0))
 (segment (start 150 80.04) (end 155.96 80.04) (width 0.3) (layer "B.Cu") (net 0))
 (segment (start 175.5 88.5) (end 175.5 101.5) (width 0.3) (layer "B.Cu") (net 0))
 (segment (start 175.5 101.5) (end 160.5 101.5) (width 0.3) (layer "B.Cu") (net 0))
 (segment (start 157.612 89.35) (end 158.591 90.329) (width 0.3) (layer "B.Cu") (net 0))
 (segment (start 158.591 90.329) (end 153.92 95) (width 0.3) (layer "B.Cu") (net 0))
 (segment (start 159.249 85.249) (end 158.591 85.249) (width 0.25) (layer "B.Cu") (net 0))
 (segment (start 141.04 89.35) (end 157.612 89.35) (width 0.3) (layer "B.Cu") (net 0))
 (segment (start 154.42 82.58) (end 150 82.58) (width 0.3) (layer "B.Cu") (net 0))
 (segment (start 175.5 72.5) (end 156 72.5) (width 0.3) (layer "B.Cu") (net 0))
 (segment (start 154.5 82.5) (end 154.42 82.58) (width 0.25) (layer "B.Cu") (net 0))
 (segment (start 176.5 83.5) (end 176.5 103) (width 0.5) (layer "B.Cu") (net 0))
 (segment (start 157.249 85.249) (end 154.5 82.5) (width 0.3) (layer "B.Cu") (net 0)))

